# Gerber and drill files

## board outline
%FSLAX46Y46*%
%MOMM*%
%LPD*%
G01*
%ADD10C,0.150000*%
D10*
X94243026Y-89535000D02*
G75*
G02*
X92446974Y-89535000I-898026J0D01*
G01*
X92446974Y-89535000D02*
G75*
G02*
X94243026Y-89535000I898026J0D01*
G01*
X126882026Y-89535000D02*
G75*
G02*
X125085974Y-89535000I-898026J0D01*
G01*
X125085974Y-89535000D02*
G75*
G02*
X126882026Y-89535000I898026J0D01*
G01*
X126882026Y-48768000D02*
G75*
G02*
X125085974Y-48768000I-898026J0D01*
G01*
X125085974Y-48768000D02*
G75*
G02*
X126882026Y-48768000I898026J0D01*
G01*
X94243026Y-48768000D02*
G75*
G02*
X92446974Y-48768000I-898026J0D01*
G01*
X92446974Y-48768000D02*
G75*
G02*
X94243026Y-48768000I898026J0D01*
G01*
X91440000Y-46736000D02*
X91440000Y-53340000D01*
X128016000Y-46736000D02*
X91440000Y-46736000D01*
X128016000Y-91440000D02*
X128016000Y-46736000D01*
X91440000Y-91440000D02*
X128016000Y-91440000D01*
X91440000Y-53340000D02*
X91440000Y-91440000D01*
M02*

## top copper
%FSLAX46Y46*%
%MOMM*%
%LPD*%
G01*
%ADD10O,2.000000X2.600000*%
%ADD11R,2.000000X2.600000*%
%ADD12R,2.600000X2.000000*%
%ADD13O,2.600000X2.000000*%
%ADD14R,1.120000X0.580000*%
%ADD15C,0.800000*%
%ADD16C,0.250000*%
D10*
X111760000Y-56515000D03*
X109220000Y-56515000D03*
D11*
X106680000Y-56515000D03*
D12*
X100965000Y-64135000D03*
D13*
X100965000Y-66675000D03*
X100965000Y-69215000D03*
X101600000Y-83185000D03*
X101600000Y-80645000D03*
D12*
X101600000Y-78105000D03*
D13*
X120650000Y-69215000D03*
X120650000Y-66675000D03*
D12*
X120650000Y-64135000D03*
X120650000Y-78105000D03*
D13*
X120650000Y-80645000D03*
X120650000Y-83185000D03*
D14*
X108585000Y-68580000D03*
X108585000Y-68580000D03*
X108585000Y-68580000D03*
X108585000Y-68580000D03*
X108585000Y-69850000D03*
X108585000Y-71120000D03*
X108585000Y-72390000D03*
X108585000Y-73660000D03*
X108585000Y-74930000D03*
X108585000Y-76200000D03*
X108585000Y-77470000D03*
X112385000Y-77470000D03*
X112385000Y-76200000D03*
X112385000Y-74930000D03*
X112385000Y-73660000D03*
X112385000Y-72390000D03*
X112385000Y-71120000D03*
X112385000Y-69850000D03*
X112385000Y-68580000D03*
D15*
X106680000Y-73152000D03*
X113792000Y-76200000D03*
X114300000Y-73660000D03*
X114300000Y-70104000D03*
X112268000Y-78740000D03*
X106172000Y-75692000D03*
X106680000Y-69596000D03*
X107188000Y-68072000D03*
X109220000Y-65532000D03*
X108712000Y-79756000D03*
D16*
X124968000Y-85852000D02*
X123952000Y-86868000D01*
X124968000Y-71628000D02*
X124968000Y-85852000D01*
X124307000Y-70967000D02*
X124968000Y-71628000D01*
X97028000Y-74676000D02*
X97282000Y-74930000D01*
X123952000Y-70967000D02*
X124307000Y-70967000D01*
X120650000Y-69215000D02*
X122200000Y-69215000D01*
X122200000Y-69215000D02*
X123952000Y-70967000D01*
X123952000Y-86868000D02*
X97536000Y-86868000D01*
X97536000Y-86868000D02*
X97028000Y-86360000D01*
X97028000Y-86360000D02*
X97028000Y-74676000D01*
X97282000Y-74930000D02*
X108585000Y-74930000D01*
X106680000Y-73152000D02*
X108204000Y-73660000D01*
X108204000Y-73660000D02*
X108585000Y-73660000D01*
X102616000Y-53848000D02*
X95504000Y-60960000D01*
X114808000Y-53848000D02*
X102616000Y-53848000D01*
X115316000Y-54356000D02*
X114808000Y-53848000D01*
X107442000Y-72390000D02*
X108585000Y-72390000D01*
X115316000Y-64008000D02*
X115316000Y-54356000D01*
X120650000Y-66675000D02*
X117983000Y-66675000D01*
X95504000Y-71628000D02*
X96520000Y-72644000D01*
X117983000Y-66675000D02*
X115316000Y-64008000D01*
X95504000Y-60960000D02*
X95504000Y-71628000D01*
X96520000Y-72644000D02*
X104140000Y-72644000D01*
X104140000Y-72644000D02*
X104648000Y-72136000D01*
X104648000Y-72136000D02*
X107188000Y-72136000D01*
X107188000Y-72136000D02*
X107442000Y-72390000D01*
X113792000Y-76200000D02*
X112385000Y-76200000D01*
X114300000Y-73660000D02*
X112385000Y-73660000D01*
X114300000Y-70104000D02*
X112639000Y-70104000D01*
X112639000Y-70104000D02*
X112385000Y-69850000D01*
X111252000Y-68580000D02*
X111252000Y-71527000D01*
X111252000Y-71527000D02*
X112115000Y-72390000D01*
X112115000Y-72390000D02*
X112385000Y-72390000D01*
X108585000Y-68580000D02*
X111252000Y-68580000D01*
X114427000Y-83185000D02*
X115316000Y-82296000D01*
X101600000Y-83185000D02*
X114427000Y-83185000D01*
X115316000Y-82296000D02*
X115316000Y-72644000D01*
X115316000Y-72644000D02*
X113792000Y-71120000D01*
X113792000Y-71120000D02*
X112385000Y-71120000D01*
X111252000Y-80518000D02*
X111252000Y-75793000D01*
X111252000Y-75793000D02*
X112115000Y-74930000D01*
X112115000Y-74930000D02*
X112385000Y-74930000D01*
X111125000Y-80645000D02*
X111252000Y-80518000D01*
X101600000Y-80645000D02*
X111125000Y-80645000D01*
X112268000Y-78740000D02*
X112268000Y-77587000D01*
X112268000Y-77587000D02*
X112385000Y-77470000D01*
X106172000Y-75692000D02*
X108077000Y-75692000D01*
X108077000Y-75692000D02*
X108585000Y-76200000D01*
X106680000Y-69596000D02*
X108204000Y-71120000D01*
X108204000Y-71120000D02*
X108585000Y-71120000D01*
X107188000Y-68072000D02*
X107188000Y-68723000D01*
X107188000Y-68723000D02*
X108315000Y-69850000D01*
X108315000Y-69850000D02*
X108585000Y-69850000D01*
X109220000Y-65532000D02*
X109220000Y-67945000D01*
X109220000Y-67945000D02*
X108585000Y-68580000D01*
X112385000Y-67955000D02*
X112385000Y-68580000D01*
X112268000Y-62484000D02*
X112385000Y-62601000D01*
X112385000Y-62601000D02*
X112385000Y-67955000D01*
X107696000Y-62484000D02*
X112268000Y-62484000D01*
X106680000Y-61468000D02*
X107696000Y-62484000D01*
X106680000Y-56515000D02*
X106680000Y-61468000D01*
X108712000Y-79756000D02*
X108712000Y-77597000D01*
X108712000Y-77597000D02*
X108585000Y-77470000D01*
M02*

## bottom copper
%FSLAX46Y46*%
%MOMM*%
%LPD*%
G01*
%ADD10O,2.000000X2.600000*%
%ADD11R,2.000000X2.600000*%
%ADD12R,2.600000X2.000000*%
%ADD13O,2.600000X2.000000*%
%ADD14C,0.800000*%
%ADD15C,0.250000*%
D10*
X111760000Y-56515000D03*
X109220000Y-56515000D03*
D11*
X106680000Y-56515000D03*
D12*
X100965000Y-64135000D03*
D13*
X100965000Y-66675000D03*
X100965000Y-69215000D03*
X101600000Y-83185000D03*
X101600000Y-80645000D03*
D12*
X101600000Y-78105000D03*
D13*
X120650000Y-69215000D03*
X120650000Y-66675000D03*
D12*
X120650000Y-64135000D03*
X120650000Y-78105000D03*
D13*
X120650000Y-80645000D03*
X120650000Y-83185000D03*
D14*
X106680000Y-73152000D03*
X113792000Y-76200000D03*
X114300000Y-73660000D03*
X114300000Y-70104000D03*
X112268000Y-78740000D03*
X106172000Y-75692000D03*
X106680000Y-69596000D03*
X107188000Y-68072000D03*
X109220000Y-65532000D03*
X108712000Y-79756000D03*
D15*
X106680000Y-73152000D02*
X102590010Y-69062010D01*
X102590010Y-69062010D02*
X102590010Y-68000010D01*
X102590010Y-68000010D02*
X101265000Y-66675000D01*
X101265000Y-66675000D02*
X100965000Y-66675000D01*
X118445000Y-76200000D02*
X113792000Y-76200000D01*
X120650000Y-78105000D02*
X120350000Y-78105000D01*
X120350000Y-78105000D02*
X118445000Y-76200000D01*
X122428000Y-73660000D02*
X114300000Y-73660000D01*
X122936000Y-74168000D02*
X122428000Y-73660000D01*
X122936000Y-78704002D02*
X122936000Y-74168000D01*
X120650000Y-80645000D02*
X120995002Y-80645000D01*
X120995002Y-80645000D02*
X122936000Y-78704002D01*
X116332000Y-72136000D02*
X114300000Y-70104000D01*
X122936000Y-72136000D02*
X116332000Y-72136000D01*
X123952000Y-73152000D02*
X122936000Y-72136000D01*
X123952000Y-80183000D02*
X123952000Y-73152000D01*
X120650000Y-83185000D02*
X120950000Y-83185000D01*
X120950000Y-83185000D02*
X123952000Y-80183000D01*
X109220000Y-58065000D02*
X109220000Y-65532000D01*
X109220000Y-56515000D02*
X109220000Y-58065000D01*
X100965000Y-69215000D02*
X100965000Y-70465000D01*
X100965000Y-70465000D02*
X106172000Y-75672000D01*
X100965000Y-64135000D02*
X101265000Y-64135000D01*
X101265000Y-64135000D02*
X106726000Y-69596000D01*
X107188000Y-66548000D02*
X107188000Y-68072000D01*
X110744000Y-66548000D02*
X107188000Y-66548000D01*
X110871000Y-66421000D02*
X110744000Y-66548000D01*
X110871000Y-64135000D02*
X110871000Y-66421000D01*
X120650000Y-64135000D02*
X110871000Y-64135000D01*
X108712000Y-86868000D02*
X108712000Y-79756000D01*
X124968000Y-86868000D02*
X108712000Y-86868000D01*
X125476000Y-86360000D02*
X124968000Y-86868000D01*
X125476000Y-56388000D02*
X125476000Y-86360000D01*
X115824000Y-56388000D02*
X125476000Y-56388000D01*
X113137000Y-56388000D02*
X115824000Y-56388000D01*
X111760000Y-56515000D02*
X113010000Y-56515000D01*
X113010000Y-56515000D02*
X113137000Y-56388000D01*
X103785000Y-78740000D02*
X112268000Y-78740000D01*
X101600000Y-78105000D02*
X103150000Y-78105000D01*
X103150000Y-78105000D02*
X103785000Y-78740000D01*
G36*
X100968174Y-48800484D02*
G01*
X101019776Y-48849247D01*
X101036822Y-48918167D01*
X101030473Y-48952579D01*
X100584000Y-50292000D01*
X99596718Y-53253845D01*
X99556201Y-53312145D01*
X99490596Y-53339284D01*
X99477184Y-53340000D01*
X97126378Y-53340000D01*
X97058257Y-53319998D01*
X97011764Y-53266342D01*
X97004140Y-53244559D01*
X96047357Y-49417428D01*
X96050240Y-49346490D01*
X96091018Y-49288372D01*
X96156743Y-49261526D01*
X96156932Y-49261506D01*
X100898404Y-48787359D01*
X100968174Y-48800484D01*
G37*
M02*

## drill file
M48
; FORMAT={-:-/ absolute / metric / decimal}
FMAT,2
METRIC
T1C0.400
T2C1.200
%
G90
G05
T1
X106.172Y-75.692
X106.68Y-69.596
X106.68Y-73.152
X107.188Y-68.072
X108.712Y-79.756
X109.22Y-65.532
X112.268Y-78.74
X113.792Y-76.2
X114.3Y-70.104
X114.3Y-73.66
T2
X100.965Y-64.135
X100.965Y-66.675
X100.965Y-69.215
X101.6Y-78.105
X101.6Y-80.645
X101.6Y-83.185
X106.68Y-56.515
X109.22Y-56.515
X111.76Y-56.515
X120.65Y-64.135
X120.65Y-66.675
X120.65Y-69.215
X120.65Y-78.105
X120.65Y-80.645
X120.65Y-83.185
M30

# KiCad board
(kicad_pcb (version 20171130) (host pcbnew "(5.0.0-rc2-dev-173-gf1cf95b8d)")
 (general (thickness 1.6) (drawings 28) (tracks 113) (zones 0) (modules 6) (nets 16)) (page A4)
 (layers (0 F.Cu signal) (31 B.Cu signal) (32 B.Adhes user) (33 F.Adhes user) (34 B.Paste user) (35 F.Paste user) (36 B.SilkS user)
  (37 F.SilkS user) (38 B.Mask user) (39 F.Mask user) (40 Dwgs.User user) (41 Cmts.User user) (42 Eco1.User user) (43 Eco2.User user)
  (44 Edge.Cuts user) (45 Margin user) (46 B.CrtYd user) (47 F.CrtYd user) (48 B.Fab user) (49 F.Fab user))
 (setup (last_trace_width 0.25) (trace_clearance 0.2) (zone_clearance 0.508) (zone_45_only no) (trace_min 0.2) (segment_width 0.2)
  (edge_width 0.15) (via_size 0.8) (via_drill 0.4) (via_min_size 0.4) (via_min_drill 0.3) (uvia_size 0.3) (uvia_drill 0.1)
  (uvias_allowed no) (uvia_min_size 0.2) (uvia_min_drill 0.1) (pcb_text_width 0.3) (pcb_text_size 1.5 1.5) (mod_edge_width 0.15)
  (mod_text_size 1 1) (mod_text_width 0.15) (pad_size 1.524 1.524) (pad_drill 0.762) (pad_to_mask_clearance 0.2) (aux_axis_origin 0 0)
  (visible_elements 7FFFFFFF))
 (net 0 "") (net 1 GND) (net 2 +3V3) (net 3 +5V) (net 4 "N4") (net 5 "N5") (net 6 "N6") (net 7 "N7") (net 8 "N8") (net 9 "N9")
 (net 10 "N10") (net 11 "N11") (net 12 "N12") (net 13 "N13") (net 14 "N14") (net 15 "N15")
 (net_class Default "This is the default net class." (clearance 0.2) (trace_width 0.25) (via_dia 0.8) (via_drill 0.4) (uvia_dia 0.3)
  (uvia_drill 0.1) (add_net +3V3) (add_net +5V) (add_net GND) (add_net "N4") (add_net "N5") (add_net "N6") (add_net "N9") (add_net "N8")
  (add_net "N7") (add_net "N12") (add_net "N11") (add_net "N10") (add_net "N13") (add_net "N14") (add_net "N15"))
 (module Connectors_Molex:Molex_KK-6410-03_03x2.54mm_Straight (layer F.Cu) (at 106.68 56.515)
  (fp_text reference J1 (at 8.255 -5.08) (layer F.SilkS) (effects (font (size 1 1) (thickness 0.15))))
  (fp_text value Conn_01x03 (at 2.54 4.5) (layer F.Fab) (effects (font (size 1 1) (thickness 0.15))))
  (pad 3 thru_hole oval (at 5.08 0) (size 2 2.6) (drill 1.2) (layers *.Cu *.Mask) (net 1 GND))
  (pad 2 thru_hole oval (at 2.54 0) (size 2 2.6) (drill 1.2) (layers *.Cu *.Mask) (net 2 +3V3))
  (pad 1 thru_hole rect (at 0 0) (size 2 2.6) (drill 1.2) (layers *.Cu *.Mask) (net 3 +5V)))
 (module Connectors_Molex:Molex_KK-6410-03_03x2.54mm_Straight (layer F.Cu) (at 100.965 64.135 270)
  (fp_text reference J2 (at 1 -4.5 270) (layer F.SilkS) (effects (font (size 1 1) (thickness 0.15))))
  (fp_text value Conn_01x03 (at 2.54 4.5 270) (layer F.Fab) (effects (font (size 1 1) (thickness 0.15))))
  (pad 1 thru_hole rect (at 0 0 270) (size 2 2.6) (drill 1.2) (layers *.Cu *.Mask) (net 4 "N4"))
  (pad 2 thru_hole oval (at 2.54 0 270) (size 2 2.6) (drill 1.2) (layers *.Cu *.Mask) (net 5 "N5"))
  (pad 3 thru_hole oval (at 5.08 0 270) (size 2 2.6) (drill 1.2) (layers *.Cu *.Mask) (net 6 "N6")))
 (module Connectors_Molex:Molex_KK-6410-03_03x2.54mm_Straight (layer F.Cu) (at 101.6 78.105 270)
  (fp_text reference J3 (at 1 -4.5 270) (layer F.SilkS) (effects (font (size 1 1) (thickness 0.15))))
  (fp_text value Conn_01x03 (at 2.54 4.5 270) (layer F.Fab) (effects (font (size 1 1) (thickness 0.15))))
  (pad 3 thru_hole oval (at 5.08 0 270) (size 2 2.6) (drill 1.2) (layers *.Cu *.Mask) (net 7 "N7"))
  (pad 2 thru_hole oval (at 2.54 0 270) (size 2 2.6) (drill 1.2) (layers *.Cu *.Mask) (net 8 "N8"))
  (pad 1 thru_hole rect (at 0 0 270) (size 2 2.6) (drill 1.2) (layers *.Cu *.Mask) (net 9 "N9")))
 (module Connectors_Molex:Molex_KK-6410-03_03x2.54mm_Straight (layer F.Cu) (at 120.65 64.135 270)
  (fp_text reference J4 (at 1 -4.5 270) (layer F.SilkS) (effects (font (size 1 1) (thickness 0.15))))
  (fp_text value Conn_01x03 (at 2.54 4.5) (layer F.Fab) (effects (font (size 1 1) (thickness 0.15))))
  (pad 3 thru_hole oval (at 5.08 0 270) (size 2 2.6) (drill 1.2) (layers *.Cu *.Mask) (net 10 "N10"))
  (pad 2 thru_hole oval (at 2.54 0 270) (size 2 2.6) (drill 1.2) (layers *.Cu *.Mask) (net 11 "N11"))
  (pad 1 thru_hole rect (at 0 0 270) (size 2 2.6) (drill 1.2) (layers *.Cu *.Mask) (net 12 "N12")))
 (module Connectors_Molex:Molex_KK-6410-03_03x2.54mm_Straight (layer F.Cu) (at 120.65 78.105 270)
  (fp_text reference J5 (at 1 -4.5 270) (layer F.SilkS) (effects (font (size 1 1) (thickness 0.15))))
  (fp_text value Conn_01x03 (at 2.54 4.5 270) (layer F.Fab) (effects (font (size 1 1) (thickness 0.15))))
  (pad 1 thru_hole rect (at 0 0 270) (size 2 2.6) (drill 1.2) (layers *.Cu *.Mask) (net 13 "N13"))
  (pad 2 thru_hole oval (at 2.54 0 270) (size 2 2.6) (drill 1.2) (layers *.Cu *.Mask) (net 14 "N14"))
  (pad 3 thru_hole oval (at 5.08 0 270) (size 2 2.6) (drill 1.2) (layers *.Cu *.Mask) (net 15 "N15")))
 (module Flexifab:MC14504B (layer F.Cu) (at 108.585 68.58)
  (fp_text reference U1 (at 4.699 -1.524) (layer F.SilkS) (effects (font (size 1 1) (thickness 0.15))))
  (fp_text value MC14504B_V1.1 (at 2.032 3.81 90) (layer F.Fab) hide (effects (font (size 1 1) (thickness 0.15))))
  (pad 1 smd rect (at 0 0) (size 1.12 0.58) (layers F.Cu F.Paste F.Mask) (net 2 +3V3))
  (pad 1 smd rect (at 0 0) (size 1.12 0.58) (layers F.Cu F.Paste F.Mask) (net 2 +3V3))
  (pad 1 smd rect (at 0 0) (size 1.12 0.58) (layers F.Cu F.Paste F.Mask) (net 2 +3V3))
  (pad 1 smd rect (at 0 0) (size 1.12 0.58) (layers F.Cu F.Paste F.Mask) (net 2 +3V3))
  (pad 2 smd rect (at 0 1.27) (size 1.12 0.58) (layers F.Cu F.Paste F.Mask) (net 12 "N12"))
  (pad 3 smd rect (at 0 2.54) (size 1.12 0.58) (layers F.Cu F.Paste F.Mask) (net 4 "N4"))
  (pad 4 smd rect (at 0 3.81) (size 1.12 0.58) (layers F.Cu F.Paste F.Mask) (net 11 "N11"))
  (pad 5 smd rect (at 0 5.08) (size 1.12 0.58) (layers F.Cu F.Paste F.Mask) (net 5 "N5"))
  (pad 6 smd rect (at 0 6.35) (size 1.12 0.58) (layers F.Cu F.Paste F.Mask) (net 10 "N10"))
  (pad 7 smd rect (at 0 7.62) (size 1.12 0.58) (layers F.Cu F.Paste F.Mask) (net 6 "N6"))
  (pad 8 smd rect (at 0 8.89) (size 1.12 0.58) (layers F.Cu F.Paste F.Mask) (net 1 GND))
  (pad 9 smd rect (at 3.8 8.89) (size 1.12 0.58) (layers F.Cu F.Paste F.Mask) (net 9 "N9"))
  (pad 10 smd rect (at 3.8 7.62) (size 1.12 0.58) (layers F.Cu F.Paste F.Mask) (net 13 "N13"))
  (pad 11 smd rect (at 3.8 6.35) (size 1.12 0.58) (layers F.Cu F.Paste F.Mask) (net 8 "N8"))
  (pad 12 smd rect (at 3.8 5.08) (size 1.12 0.58) (layers F.Cu F.Paste F.Mask) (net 14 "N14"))
  (pad 13 smd rect (at 3.8 3.81) (size 1.12 0.58) (layers F.Cu F.Paste F.Mask) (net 2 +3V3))
  (pad 14 smd rect (at 3.8 2.54) (size 1.12 0.58) (layers F.Cu F.Paste F.Mask) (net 7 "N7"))
  (pad 15 smd rect (at 3.8 1.27) (size 1.12 0.58) (layers F.Cu F.Paste F.Mask) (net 15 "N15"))
  (pad 16 smd rect (at 3.8 0) (size 1.12 0.58) (layers F.Cu F.Paste F.Mask) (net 3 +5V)))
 (gr_circle (center 93.345 89.535) (end 93.98 90.17) (layer Edge.Cuts) (width 0.15))
 (gr_circle (center 125.984 89.535) (end 126.619 90.17) (layer Edge.Cuts) (width 0.15))
 (gr_circle (center 125.984 48.768) (end 126.619 49.403) (layer Edge.Cuts) (width 0.15))
 (gr_circle (center 93.345 48.768) (end 93.98 49.403) (layer Edge.Cuts) (width 0.15))
 (gr_line (start 91.44 46.736) (end 91.44 53.34) (layer Edge.Cuts) (width 0.15))
 (gr_line (start 128.016 46.736) (end 91.44 46.736) (layer Edge.Cuts) (width 0.15))
 (gr_line (start 128.016 91.44) (end 128.016 46.736) (layer Edge.Cuts) (width 0.15))
 (gr_line (start 91.44 91.44) (end 128.016 91.44) (layer Edge.Cuts) (width 0.15))
 (gr_line (start 91.44 53.34) (end 91.44 91.44) (layer Edge.Cuts) (width 0.15))
 (segment (start 124.968 85.852) (end 123.952 86.868) (width 0.25) (layer F.Cu) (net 10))
 (segment (start 124.968 71.628) (end 124.968 85.852) (width 0.25) (layer F.Cu) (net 10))
 (segment (start 124.307 70.967) (end 124.968 71.628) (width 0.25) (layer F.Cu) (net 10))
 (segment (start 97.028 74.676) (end 97.282 74.93) (width 0.25) (layer F.Cu) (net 10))
 (segment (start 123.952 70.967) (end 124.307 70.967) (width 0.25) (layer F.Cu) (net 10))
 (segment (start 120.65 69.215) (end 122.2 69.215) (width 0.25) (layer F.Cu) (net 10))
 (segment (start 122.2 69.215) (end 123.952 70.967) (width 0.25) (layer F.Cu) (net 10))
 (segment (start 123.952 86.868) (end 97.536 86.868) (width 0.25) (layer F.Cu) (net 10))
 (segment (start 97.536 86.868) (end 97.028 86.36) (width 0.25) (layer F.Cu) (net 10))
 (segment (start 97.028 86.36) (end 97.028 74.676) (width 0.25) (layer F.Cu) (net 10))
 (segment (start 97.282 74.93) (end 108.585 74.93) (width 0.25) (layer F.Cu) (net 10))
 (segment (start 106.68 73.152) (end 102.59001 69.06201) (width 0.25) (layer B.Cu) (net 5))
 (segment (start 102.59001 69.06201) (end 102.59001 68.00001) (width 0.25) (layer B.Cu) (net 5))
 (segment (start 102.59001 68.00001) (end 101.265 66.675) (width 0.25) (layer B.Cu) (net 5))
 (segment (start 101.265 66.675) (end 100.965 66.675) (width 0.25) (layer B.Cu) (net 5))
 (segment (start 106.68 73.152) (end 108.204 73.66) (width 0.25) (layer F.Cu) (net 5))
 (via (at 106.68 73.152) (size 0.8) (drill 0.4) (layers F.Cu B.Cu) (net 5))
 (segment (start 108.204 73.66) (end 108.585 73.66) (width 0.25) (layer F.Cu) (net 5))
 (segment (start 102.616 53.848) (end 95.504 60.96) (width 0.25) (layer F.Cu) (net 11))
 (segment (start 114.808 53.848) (end 102.616 53.848) (width 0.25) (layer F.Cu) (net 11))
 (segment (start 115.316 54.356) (end 114.808 53.848) (width 0.25) (layer F.Cu) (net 11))
 (segment (start 107.442 72.39) (end 108.585 72.39) (width 0.25) (layer F.Cu) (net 11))
 (segment (start 115.316 64.008) (end 115.316 54.356) (width 0.25) (layer F.Cu) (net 11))
 (segment (start 120.65 66.675) (end 117.983 66.675) (width 0.25) (layer F.Cu) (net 11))
 (segment (start 95.504 71.628) (end 96.52 72.644) (width 0.25) (layer F.Cu) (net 11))
 (segment (start 117.983 66.675) (end 115.316 64.008) (width 0.25) (layer F.Cu) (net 11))
 (segment (start 95.504 60.96) (end 95.504 71.628) (width 0.25) (layer F.Cu) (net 11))
 (segment (start 96.52 72.644) (end 104.14 72.644) (width 0.25) (layer F.Cu) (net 11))
 (segment (start 104.14 72.644) (end 104.648 72.136) (width 0.25) (layer F.Cu) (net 11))
 (segment (start 104.648 72.136) (end 107.188 72.136) (width 0.25) (layer F.Cu) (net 11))
 (segment (start 107.188 72.136) (end 107.442 72.39) (width 0.25) (layer F.Cu) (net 11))
 (segment (start 113.792 76.2) (end 112.385 76.2) (width 0.25) (layer F.Cu) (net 13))
 (via (at 113.792 76.2) (size 0.8) (drill 0.4) (layers F.Cu B.Cu) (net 13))
 (segment (start 114.3 73.66) (end 112.385 73.66) (width 0.25) (layer F.Cu) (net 14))
 (via (at 114.3 73.66) (size 0.8) (drill 0.4) (layers F.Cu B.Cu) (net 14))
 (segment (start 114.3 70.104) (end 112.639 70.104) (width 0.25) (layer F.Cu) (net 15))
 (segment (start 112.639 70.104) (end 112.385 69.85) (width 0.25) (layer F.Cu) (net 15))
 (via (at 114.3 70.104) (size 0.8) (drill 0.4) (layers F.Cu B.Cu) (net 15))
 (segment (start 111.252 68.58) (end 111.252 71.527) (width 0.25) (layer F.Cu) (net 2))
 (segment (start 111.252 71.527) (end 112.115 72.39) (width 0.25) (layer F.Cu) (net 2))
 (segment (start 112.115 72.39) (end 112.385 72.39) (width 0.25) (layer F.Cu) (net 2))
 (segment (start 108.585 68.58) (end 111.252 68.58) (width 0.25) (layer F.Cu) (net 2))
 (segment (start 118.445 76.2) (end 113.792 76.2) (width 0.25) (layer B.Cu) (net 13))
 (segment (start 120.65 78.105) (end 120.35 78.105) (width 0.25) (layer B.Cu) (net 13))
 (segment (start 120.35 78.105) (end 118.445 76.2) (width 0.25) (layer B.Cu) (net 13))
 (segment (start 122.428 73.66) (end 114.3 73.66) (width 0.25) (layer B.Cu) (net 14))
 (segment (start 122.936 74.168) (end 122.428 73.66) (width 0.25) (layer B.Cu) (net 14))
 (segment (start 122.936 78.704002) (end 122.936 74.168) (width 0.25) (layer B.Cu) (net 14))
 (segment (start 120.65 80.645) (end 120.995002 80.645) (width 0.25) (layer B.Cu) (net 14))
 (segment (start 120.995002 80.645) (end 122.936 78.704002) (width 0.25) (layer B.Cu) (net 14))
 (segment (start 116.332 72.136) (end 114.3 70.104) (width 0.25) (layer B.Cu) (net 15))
 (segment (start 122.936 72.136) (end 116.332 72.136) (width 0.25) (layer B.Cu) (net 15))
 (segment (start 123.952 73.152) (end 122.936 72.136) (width 0.25) (layer B.Cu) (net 15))
 (segment (start 123.952 80.183) (end 123.952 73.152) (width 0.25) (layer B.Cu) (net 15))
 (segment (start 120.65 83.185) (end 120.95 83.185) (width 0.25) (layer B.Cu) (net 15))
 (segment (start 120.95 83.185) (end 123.952 80.183) (width 0.25) (layer B.Cu) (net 15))
 (segment (start 114.427 83.185) (end 115.316 82.296) (width 0.25) (layer F.Cu) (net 7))
 (segment (start 101.6 83.185) (end 114.427 83.185) (width 0.25) (layer F.Cu) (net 7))
 (segment (start 115.316 82.296) (end 115.316 72.644) (width 0.25) (layer F.Cu) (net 7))
 (segment (start 115.316 72.644) (end 113.792 71.12) (width 0.25) (layer F.Cu) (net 7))
 (segment (start 113.792 71.12) (end 112.385 71.12) (width 0.25) (layer F.Cu) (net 7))
 (segment (start 111.252 80.518) (end 111.252 75.793) (width 0.25) (layer F.Cu) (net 8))
 (segment (start 111.252 75.793) (end 112.115 74.93) (width 0.25) (layer F.Cu) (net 8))
 (segment (start 112.115 74.93) (end 112.385 74.93) (width 0.25) (layer F.Cu) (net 8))
 (segment (start 111.125 80.645) (end 111.252 80.518) (width 0.25) (layer F.Cu) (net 8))
 (segment (start 101.6 80.645) (end 111.125 80.645) (width 0.25) (layer F.Cu) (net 8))
 (segment (start 112.268 78.74) (end 112.268 77.587) (width 0.25) (layer F.Cu) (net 9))
 (segment (start 112.268 77.587) (end 112.385 77.47) (width 0.25) (layer F.Cu) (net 9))
 (via (at 112.268 78.74) (size 0.8) (drill 0.4) (layers F.Cu B.Cu) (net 9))
 (segment (start 106.172 75.692) (end 108.077 75.692) (width 0.25) (layer F.Cu) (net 6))
 (segment (start 108.077 75.692) (end 108.585 76.2) (width 0.25) (layer F.Cu) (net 6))
 (via (at 106.172 75.692) (size 0.8) (drill 0.4) (layers F.Cu B.Cu) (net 6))
 (segment (start 106.68 69.596) (end 108.204 71.12) (width 0.25) (layer F.Cu) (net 4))
 (segment (start 108.204 71.12) (end 108.585 71.12) (width 0.25) (layer F.Cu) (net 4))
 (via (at 106.68 69.596) (size 0.8) (drill 0.4) (layers F.Cu B.Cu) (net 4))
 (segment (start 107.188 68.072) (end 107.188 68.723) (width 0.25) (layer F.Cu) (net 12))
 (segment (start 107.188 68.723) (end 108.315 69.85) (width 0.25) (layer F.Cu) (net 12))
 (segment (start 108.315 69.85) (end 108.585 69.85) (width 0.25) (layer F.Cu) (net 12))
 (via (at 107.188 68.072) (size 0.8) (drill 0.4) (layers F.Cu B.Cu) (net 12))
 (segment (start 109.22 65.532) (end 109.22 67.945) (width 0.25) (layer F.Cu) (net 2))
 (segment (start 109.22 67.945) (end 108.585 68.58) (width 0.25) (layer F.Cu) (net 2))
 (via (at 109.22 65.532) (size 0.8) (drill 0.4) (layers F.Cu B.Cu) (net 2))
 (segment (start 109.22 58.065) (end 109.22 65.532) (width 0.25) (layer B.Cu) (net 2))
 (segment (start 109.22 56.515) (end 109.22 58.065) (width 0.25) (layer B.Cu) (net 2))
 (segment (start 100.965 69.215) (end 100.965 70.465) (width 0.25) (layer B.Cu) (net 6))
 (segment (start 100.965 70.465) (end 106.172 75.672) (width 0.25) (layer B.Cu) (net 6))
 (segment (start 100.965 64.135) (end 101.265 64.135) (width 0.25) (layer B.Cu) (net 4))
 (segment (start 101.265 64.135) (end 106.726 69.596) (width 0.25) (layer B.Cu) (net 4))
 (segment (start 112.385 67.955) (end 112.385 68.58) (width 0.25) (layer F.Cu) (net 3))
 (segment (start 112.268 62.484) (end 112.385 62.601) (width 0.25) (layer F.Cu) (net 3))
 (segment (start 112.385 62.601) (end 112.385 67.955) (width 0.25) (layer F.Cu) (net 3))
 (segment (start 107.696 62.484) (end 112.268 62.484) (width 0.25) (layer F.Cu) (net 3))
 (segment (start 106.68 61.468) (end 107.696 62.484) (width 0.25) (layer F.Cu) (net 3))
 (segment (start 106.68 56.515) (end 106.68 61.468) (width 0.25) (layer F.Cu) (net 3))
 (segment (start 107.188 66.548) (end 107.188 68.072) (width 0.25) (layer B.Cu) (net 12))
 (segment (start 110.744 66.548) (end 107.188 66.548) (width 0.25) (layer B.Cu) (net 12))
 (segment (start 110.871 66.421) (end 110.744 66.548) (width 0.25) (layer B.Cu) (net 12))
 (segment (start 110.871 64.135) (end 110.871 66.421) (width 0.25) (layer B.Cu) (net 12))
 (segment (start 120.65 64.135) (end 110.871 64.135) (width 0.25) (layer B.Cu) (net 12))
 (segment (start 108.712 79.756) (end 108.712 77.597) (width 0.25) (layer F.Cu) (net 1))
 (segment (start 108.712 77.597) (end 108.585 77.47) (width 0.25) (layer F.Cu) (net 1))
 (via (at 108.712 79.756) (size 0.8) (drill 0.4) (layers F.Cu B.Cu) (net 1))
 (segment (start 108.712 86.868) (end 108.712 79.756) (width 0.25) (layer B.Cu) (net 1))
 (segment (start 124.968 86.868) (end 108.712 86.868) (width 0.25) (layer B.Cu) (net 1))
 (segment (start 125.476 86.36) (end 124.968 86.868) (width 0.25) (layer B.Cu) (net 1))
 (segment (start 125.476 56.388) (end 125.476 86.36) (width 0.25) (layer B.Cu) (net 1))
 (segment (start 115.824 56.388) (end 125.476 56.388) (width 0.25) (layer B.Cu) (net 1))
 (segment (start 113.137 56.388) (end 115.824 56.388) (width 0.25) (layer B.Cu) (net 1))
 (segment (start 111.76 56.515) (end 113.01 56.515) (width 0.25) (layer B.Cu) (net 1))
 (segment (start 113.01 56.515) (end 113.137 56.388) (width 0.25) (layer B.Cu) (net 1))
 (segment (start 103.785 78.74) (end 112.268 78.74) (width 0.25) (layer B.Cu) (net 9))
 (segment (start 101.6 78.105) (end 103.15 78.105) (width 0.25) (layer B.Cu) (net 9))
 (segment (start 103.15 78.105) (end 103.785 78.74) (width 0.25) (layer B.Cu) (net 9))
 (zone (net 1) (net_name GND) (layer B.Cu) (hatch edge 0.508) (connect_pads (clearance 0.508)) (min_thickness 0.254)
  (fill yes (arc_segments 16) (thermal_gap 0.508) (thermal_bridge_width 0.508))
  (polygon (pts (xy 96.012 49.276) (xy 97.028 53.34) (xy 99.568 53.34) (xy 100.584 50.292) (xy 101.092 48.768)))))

